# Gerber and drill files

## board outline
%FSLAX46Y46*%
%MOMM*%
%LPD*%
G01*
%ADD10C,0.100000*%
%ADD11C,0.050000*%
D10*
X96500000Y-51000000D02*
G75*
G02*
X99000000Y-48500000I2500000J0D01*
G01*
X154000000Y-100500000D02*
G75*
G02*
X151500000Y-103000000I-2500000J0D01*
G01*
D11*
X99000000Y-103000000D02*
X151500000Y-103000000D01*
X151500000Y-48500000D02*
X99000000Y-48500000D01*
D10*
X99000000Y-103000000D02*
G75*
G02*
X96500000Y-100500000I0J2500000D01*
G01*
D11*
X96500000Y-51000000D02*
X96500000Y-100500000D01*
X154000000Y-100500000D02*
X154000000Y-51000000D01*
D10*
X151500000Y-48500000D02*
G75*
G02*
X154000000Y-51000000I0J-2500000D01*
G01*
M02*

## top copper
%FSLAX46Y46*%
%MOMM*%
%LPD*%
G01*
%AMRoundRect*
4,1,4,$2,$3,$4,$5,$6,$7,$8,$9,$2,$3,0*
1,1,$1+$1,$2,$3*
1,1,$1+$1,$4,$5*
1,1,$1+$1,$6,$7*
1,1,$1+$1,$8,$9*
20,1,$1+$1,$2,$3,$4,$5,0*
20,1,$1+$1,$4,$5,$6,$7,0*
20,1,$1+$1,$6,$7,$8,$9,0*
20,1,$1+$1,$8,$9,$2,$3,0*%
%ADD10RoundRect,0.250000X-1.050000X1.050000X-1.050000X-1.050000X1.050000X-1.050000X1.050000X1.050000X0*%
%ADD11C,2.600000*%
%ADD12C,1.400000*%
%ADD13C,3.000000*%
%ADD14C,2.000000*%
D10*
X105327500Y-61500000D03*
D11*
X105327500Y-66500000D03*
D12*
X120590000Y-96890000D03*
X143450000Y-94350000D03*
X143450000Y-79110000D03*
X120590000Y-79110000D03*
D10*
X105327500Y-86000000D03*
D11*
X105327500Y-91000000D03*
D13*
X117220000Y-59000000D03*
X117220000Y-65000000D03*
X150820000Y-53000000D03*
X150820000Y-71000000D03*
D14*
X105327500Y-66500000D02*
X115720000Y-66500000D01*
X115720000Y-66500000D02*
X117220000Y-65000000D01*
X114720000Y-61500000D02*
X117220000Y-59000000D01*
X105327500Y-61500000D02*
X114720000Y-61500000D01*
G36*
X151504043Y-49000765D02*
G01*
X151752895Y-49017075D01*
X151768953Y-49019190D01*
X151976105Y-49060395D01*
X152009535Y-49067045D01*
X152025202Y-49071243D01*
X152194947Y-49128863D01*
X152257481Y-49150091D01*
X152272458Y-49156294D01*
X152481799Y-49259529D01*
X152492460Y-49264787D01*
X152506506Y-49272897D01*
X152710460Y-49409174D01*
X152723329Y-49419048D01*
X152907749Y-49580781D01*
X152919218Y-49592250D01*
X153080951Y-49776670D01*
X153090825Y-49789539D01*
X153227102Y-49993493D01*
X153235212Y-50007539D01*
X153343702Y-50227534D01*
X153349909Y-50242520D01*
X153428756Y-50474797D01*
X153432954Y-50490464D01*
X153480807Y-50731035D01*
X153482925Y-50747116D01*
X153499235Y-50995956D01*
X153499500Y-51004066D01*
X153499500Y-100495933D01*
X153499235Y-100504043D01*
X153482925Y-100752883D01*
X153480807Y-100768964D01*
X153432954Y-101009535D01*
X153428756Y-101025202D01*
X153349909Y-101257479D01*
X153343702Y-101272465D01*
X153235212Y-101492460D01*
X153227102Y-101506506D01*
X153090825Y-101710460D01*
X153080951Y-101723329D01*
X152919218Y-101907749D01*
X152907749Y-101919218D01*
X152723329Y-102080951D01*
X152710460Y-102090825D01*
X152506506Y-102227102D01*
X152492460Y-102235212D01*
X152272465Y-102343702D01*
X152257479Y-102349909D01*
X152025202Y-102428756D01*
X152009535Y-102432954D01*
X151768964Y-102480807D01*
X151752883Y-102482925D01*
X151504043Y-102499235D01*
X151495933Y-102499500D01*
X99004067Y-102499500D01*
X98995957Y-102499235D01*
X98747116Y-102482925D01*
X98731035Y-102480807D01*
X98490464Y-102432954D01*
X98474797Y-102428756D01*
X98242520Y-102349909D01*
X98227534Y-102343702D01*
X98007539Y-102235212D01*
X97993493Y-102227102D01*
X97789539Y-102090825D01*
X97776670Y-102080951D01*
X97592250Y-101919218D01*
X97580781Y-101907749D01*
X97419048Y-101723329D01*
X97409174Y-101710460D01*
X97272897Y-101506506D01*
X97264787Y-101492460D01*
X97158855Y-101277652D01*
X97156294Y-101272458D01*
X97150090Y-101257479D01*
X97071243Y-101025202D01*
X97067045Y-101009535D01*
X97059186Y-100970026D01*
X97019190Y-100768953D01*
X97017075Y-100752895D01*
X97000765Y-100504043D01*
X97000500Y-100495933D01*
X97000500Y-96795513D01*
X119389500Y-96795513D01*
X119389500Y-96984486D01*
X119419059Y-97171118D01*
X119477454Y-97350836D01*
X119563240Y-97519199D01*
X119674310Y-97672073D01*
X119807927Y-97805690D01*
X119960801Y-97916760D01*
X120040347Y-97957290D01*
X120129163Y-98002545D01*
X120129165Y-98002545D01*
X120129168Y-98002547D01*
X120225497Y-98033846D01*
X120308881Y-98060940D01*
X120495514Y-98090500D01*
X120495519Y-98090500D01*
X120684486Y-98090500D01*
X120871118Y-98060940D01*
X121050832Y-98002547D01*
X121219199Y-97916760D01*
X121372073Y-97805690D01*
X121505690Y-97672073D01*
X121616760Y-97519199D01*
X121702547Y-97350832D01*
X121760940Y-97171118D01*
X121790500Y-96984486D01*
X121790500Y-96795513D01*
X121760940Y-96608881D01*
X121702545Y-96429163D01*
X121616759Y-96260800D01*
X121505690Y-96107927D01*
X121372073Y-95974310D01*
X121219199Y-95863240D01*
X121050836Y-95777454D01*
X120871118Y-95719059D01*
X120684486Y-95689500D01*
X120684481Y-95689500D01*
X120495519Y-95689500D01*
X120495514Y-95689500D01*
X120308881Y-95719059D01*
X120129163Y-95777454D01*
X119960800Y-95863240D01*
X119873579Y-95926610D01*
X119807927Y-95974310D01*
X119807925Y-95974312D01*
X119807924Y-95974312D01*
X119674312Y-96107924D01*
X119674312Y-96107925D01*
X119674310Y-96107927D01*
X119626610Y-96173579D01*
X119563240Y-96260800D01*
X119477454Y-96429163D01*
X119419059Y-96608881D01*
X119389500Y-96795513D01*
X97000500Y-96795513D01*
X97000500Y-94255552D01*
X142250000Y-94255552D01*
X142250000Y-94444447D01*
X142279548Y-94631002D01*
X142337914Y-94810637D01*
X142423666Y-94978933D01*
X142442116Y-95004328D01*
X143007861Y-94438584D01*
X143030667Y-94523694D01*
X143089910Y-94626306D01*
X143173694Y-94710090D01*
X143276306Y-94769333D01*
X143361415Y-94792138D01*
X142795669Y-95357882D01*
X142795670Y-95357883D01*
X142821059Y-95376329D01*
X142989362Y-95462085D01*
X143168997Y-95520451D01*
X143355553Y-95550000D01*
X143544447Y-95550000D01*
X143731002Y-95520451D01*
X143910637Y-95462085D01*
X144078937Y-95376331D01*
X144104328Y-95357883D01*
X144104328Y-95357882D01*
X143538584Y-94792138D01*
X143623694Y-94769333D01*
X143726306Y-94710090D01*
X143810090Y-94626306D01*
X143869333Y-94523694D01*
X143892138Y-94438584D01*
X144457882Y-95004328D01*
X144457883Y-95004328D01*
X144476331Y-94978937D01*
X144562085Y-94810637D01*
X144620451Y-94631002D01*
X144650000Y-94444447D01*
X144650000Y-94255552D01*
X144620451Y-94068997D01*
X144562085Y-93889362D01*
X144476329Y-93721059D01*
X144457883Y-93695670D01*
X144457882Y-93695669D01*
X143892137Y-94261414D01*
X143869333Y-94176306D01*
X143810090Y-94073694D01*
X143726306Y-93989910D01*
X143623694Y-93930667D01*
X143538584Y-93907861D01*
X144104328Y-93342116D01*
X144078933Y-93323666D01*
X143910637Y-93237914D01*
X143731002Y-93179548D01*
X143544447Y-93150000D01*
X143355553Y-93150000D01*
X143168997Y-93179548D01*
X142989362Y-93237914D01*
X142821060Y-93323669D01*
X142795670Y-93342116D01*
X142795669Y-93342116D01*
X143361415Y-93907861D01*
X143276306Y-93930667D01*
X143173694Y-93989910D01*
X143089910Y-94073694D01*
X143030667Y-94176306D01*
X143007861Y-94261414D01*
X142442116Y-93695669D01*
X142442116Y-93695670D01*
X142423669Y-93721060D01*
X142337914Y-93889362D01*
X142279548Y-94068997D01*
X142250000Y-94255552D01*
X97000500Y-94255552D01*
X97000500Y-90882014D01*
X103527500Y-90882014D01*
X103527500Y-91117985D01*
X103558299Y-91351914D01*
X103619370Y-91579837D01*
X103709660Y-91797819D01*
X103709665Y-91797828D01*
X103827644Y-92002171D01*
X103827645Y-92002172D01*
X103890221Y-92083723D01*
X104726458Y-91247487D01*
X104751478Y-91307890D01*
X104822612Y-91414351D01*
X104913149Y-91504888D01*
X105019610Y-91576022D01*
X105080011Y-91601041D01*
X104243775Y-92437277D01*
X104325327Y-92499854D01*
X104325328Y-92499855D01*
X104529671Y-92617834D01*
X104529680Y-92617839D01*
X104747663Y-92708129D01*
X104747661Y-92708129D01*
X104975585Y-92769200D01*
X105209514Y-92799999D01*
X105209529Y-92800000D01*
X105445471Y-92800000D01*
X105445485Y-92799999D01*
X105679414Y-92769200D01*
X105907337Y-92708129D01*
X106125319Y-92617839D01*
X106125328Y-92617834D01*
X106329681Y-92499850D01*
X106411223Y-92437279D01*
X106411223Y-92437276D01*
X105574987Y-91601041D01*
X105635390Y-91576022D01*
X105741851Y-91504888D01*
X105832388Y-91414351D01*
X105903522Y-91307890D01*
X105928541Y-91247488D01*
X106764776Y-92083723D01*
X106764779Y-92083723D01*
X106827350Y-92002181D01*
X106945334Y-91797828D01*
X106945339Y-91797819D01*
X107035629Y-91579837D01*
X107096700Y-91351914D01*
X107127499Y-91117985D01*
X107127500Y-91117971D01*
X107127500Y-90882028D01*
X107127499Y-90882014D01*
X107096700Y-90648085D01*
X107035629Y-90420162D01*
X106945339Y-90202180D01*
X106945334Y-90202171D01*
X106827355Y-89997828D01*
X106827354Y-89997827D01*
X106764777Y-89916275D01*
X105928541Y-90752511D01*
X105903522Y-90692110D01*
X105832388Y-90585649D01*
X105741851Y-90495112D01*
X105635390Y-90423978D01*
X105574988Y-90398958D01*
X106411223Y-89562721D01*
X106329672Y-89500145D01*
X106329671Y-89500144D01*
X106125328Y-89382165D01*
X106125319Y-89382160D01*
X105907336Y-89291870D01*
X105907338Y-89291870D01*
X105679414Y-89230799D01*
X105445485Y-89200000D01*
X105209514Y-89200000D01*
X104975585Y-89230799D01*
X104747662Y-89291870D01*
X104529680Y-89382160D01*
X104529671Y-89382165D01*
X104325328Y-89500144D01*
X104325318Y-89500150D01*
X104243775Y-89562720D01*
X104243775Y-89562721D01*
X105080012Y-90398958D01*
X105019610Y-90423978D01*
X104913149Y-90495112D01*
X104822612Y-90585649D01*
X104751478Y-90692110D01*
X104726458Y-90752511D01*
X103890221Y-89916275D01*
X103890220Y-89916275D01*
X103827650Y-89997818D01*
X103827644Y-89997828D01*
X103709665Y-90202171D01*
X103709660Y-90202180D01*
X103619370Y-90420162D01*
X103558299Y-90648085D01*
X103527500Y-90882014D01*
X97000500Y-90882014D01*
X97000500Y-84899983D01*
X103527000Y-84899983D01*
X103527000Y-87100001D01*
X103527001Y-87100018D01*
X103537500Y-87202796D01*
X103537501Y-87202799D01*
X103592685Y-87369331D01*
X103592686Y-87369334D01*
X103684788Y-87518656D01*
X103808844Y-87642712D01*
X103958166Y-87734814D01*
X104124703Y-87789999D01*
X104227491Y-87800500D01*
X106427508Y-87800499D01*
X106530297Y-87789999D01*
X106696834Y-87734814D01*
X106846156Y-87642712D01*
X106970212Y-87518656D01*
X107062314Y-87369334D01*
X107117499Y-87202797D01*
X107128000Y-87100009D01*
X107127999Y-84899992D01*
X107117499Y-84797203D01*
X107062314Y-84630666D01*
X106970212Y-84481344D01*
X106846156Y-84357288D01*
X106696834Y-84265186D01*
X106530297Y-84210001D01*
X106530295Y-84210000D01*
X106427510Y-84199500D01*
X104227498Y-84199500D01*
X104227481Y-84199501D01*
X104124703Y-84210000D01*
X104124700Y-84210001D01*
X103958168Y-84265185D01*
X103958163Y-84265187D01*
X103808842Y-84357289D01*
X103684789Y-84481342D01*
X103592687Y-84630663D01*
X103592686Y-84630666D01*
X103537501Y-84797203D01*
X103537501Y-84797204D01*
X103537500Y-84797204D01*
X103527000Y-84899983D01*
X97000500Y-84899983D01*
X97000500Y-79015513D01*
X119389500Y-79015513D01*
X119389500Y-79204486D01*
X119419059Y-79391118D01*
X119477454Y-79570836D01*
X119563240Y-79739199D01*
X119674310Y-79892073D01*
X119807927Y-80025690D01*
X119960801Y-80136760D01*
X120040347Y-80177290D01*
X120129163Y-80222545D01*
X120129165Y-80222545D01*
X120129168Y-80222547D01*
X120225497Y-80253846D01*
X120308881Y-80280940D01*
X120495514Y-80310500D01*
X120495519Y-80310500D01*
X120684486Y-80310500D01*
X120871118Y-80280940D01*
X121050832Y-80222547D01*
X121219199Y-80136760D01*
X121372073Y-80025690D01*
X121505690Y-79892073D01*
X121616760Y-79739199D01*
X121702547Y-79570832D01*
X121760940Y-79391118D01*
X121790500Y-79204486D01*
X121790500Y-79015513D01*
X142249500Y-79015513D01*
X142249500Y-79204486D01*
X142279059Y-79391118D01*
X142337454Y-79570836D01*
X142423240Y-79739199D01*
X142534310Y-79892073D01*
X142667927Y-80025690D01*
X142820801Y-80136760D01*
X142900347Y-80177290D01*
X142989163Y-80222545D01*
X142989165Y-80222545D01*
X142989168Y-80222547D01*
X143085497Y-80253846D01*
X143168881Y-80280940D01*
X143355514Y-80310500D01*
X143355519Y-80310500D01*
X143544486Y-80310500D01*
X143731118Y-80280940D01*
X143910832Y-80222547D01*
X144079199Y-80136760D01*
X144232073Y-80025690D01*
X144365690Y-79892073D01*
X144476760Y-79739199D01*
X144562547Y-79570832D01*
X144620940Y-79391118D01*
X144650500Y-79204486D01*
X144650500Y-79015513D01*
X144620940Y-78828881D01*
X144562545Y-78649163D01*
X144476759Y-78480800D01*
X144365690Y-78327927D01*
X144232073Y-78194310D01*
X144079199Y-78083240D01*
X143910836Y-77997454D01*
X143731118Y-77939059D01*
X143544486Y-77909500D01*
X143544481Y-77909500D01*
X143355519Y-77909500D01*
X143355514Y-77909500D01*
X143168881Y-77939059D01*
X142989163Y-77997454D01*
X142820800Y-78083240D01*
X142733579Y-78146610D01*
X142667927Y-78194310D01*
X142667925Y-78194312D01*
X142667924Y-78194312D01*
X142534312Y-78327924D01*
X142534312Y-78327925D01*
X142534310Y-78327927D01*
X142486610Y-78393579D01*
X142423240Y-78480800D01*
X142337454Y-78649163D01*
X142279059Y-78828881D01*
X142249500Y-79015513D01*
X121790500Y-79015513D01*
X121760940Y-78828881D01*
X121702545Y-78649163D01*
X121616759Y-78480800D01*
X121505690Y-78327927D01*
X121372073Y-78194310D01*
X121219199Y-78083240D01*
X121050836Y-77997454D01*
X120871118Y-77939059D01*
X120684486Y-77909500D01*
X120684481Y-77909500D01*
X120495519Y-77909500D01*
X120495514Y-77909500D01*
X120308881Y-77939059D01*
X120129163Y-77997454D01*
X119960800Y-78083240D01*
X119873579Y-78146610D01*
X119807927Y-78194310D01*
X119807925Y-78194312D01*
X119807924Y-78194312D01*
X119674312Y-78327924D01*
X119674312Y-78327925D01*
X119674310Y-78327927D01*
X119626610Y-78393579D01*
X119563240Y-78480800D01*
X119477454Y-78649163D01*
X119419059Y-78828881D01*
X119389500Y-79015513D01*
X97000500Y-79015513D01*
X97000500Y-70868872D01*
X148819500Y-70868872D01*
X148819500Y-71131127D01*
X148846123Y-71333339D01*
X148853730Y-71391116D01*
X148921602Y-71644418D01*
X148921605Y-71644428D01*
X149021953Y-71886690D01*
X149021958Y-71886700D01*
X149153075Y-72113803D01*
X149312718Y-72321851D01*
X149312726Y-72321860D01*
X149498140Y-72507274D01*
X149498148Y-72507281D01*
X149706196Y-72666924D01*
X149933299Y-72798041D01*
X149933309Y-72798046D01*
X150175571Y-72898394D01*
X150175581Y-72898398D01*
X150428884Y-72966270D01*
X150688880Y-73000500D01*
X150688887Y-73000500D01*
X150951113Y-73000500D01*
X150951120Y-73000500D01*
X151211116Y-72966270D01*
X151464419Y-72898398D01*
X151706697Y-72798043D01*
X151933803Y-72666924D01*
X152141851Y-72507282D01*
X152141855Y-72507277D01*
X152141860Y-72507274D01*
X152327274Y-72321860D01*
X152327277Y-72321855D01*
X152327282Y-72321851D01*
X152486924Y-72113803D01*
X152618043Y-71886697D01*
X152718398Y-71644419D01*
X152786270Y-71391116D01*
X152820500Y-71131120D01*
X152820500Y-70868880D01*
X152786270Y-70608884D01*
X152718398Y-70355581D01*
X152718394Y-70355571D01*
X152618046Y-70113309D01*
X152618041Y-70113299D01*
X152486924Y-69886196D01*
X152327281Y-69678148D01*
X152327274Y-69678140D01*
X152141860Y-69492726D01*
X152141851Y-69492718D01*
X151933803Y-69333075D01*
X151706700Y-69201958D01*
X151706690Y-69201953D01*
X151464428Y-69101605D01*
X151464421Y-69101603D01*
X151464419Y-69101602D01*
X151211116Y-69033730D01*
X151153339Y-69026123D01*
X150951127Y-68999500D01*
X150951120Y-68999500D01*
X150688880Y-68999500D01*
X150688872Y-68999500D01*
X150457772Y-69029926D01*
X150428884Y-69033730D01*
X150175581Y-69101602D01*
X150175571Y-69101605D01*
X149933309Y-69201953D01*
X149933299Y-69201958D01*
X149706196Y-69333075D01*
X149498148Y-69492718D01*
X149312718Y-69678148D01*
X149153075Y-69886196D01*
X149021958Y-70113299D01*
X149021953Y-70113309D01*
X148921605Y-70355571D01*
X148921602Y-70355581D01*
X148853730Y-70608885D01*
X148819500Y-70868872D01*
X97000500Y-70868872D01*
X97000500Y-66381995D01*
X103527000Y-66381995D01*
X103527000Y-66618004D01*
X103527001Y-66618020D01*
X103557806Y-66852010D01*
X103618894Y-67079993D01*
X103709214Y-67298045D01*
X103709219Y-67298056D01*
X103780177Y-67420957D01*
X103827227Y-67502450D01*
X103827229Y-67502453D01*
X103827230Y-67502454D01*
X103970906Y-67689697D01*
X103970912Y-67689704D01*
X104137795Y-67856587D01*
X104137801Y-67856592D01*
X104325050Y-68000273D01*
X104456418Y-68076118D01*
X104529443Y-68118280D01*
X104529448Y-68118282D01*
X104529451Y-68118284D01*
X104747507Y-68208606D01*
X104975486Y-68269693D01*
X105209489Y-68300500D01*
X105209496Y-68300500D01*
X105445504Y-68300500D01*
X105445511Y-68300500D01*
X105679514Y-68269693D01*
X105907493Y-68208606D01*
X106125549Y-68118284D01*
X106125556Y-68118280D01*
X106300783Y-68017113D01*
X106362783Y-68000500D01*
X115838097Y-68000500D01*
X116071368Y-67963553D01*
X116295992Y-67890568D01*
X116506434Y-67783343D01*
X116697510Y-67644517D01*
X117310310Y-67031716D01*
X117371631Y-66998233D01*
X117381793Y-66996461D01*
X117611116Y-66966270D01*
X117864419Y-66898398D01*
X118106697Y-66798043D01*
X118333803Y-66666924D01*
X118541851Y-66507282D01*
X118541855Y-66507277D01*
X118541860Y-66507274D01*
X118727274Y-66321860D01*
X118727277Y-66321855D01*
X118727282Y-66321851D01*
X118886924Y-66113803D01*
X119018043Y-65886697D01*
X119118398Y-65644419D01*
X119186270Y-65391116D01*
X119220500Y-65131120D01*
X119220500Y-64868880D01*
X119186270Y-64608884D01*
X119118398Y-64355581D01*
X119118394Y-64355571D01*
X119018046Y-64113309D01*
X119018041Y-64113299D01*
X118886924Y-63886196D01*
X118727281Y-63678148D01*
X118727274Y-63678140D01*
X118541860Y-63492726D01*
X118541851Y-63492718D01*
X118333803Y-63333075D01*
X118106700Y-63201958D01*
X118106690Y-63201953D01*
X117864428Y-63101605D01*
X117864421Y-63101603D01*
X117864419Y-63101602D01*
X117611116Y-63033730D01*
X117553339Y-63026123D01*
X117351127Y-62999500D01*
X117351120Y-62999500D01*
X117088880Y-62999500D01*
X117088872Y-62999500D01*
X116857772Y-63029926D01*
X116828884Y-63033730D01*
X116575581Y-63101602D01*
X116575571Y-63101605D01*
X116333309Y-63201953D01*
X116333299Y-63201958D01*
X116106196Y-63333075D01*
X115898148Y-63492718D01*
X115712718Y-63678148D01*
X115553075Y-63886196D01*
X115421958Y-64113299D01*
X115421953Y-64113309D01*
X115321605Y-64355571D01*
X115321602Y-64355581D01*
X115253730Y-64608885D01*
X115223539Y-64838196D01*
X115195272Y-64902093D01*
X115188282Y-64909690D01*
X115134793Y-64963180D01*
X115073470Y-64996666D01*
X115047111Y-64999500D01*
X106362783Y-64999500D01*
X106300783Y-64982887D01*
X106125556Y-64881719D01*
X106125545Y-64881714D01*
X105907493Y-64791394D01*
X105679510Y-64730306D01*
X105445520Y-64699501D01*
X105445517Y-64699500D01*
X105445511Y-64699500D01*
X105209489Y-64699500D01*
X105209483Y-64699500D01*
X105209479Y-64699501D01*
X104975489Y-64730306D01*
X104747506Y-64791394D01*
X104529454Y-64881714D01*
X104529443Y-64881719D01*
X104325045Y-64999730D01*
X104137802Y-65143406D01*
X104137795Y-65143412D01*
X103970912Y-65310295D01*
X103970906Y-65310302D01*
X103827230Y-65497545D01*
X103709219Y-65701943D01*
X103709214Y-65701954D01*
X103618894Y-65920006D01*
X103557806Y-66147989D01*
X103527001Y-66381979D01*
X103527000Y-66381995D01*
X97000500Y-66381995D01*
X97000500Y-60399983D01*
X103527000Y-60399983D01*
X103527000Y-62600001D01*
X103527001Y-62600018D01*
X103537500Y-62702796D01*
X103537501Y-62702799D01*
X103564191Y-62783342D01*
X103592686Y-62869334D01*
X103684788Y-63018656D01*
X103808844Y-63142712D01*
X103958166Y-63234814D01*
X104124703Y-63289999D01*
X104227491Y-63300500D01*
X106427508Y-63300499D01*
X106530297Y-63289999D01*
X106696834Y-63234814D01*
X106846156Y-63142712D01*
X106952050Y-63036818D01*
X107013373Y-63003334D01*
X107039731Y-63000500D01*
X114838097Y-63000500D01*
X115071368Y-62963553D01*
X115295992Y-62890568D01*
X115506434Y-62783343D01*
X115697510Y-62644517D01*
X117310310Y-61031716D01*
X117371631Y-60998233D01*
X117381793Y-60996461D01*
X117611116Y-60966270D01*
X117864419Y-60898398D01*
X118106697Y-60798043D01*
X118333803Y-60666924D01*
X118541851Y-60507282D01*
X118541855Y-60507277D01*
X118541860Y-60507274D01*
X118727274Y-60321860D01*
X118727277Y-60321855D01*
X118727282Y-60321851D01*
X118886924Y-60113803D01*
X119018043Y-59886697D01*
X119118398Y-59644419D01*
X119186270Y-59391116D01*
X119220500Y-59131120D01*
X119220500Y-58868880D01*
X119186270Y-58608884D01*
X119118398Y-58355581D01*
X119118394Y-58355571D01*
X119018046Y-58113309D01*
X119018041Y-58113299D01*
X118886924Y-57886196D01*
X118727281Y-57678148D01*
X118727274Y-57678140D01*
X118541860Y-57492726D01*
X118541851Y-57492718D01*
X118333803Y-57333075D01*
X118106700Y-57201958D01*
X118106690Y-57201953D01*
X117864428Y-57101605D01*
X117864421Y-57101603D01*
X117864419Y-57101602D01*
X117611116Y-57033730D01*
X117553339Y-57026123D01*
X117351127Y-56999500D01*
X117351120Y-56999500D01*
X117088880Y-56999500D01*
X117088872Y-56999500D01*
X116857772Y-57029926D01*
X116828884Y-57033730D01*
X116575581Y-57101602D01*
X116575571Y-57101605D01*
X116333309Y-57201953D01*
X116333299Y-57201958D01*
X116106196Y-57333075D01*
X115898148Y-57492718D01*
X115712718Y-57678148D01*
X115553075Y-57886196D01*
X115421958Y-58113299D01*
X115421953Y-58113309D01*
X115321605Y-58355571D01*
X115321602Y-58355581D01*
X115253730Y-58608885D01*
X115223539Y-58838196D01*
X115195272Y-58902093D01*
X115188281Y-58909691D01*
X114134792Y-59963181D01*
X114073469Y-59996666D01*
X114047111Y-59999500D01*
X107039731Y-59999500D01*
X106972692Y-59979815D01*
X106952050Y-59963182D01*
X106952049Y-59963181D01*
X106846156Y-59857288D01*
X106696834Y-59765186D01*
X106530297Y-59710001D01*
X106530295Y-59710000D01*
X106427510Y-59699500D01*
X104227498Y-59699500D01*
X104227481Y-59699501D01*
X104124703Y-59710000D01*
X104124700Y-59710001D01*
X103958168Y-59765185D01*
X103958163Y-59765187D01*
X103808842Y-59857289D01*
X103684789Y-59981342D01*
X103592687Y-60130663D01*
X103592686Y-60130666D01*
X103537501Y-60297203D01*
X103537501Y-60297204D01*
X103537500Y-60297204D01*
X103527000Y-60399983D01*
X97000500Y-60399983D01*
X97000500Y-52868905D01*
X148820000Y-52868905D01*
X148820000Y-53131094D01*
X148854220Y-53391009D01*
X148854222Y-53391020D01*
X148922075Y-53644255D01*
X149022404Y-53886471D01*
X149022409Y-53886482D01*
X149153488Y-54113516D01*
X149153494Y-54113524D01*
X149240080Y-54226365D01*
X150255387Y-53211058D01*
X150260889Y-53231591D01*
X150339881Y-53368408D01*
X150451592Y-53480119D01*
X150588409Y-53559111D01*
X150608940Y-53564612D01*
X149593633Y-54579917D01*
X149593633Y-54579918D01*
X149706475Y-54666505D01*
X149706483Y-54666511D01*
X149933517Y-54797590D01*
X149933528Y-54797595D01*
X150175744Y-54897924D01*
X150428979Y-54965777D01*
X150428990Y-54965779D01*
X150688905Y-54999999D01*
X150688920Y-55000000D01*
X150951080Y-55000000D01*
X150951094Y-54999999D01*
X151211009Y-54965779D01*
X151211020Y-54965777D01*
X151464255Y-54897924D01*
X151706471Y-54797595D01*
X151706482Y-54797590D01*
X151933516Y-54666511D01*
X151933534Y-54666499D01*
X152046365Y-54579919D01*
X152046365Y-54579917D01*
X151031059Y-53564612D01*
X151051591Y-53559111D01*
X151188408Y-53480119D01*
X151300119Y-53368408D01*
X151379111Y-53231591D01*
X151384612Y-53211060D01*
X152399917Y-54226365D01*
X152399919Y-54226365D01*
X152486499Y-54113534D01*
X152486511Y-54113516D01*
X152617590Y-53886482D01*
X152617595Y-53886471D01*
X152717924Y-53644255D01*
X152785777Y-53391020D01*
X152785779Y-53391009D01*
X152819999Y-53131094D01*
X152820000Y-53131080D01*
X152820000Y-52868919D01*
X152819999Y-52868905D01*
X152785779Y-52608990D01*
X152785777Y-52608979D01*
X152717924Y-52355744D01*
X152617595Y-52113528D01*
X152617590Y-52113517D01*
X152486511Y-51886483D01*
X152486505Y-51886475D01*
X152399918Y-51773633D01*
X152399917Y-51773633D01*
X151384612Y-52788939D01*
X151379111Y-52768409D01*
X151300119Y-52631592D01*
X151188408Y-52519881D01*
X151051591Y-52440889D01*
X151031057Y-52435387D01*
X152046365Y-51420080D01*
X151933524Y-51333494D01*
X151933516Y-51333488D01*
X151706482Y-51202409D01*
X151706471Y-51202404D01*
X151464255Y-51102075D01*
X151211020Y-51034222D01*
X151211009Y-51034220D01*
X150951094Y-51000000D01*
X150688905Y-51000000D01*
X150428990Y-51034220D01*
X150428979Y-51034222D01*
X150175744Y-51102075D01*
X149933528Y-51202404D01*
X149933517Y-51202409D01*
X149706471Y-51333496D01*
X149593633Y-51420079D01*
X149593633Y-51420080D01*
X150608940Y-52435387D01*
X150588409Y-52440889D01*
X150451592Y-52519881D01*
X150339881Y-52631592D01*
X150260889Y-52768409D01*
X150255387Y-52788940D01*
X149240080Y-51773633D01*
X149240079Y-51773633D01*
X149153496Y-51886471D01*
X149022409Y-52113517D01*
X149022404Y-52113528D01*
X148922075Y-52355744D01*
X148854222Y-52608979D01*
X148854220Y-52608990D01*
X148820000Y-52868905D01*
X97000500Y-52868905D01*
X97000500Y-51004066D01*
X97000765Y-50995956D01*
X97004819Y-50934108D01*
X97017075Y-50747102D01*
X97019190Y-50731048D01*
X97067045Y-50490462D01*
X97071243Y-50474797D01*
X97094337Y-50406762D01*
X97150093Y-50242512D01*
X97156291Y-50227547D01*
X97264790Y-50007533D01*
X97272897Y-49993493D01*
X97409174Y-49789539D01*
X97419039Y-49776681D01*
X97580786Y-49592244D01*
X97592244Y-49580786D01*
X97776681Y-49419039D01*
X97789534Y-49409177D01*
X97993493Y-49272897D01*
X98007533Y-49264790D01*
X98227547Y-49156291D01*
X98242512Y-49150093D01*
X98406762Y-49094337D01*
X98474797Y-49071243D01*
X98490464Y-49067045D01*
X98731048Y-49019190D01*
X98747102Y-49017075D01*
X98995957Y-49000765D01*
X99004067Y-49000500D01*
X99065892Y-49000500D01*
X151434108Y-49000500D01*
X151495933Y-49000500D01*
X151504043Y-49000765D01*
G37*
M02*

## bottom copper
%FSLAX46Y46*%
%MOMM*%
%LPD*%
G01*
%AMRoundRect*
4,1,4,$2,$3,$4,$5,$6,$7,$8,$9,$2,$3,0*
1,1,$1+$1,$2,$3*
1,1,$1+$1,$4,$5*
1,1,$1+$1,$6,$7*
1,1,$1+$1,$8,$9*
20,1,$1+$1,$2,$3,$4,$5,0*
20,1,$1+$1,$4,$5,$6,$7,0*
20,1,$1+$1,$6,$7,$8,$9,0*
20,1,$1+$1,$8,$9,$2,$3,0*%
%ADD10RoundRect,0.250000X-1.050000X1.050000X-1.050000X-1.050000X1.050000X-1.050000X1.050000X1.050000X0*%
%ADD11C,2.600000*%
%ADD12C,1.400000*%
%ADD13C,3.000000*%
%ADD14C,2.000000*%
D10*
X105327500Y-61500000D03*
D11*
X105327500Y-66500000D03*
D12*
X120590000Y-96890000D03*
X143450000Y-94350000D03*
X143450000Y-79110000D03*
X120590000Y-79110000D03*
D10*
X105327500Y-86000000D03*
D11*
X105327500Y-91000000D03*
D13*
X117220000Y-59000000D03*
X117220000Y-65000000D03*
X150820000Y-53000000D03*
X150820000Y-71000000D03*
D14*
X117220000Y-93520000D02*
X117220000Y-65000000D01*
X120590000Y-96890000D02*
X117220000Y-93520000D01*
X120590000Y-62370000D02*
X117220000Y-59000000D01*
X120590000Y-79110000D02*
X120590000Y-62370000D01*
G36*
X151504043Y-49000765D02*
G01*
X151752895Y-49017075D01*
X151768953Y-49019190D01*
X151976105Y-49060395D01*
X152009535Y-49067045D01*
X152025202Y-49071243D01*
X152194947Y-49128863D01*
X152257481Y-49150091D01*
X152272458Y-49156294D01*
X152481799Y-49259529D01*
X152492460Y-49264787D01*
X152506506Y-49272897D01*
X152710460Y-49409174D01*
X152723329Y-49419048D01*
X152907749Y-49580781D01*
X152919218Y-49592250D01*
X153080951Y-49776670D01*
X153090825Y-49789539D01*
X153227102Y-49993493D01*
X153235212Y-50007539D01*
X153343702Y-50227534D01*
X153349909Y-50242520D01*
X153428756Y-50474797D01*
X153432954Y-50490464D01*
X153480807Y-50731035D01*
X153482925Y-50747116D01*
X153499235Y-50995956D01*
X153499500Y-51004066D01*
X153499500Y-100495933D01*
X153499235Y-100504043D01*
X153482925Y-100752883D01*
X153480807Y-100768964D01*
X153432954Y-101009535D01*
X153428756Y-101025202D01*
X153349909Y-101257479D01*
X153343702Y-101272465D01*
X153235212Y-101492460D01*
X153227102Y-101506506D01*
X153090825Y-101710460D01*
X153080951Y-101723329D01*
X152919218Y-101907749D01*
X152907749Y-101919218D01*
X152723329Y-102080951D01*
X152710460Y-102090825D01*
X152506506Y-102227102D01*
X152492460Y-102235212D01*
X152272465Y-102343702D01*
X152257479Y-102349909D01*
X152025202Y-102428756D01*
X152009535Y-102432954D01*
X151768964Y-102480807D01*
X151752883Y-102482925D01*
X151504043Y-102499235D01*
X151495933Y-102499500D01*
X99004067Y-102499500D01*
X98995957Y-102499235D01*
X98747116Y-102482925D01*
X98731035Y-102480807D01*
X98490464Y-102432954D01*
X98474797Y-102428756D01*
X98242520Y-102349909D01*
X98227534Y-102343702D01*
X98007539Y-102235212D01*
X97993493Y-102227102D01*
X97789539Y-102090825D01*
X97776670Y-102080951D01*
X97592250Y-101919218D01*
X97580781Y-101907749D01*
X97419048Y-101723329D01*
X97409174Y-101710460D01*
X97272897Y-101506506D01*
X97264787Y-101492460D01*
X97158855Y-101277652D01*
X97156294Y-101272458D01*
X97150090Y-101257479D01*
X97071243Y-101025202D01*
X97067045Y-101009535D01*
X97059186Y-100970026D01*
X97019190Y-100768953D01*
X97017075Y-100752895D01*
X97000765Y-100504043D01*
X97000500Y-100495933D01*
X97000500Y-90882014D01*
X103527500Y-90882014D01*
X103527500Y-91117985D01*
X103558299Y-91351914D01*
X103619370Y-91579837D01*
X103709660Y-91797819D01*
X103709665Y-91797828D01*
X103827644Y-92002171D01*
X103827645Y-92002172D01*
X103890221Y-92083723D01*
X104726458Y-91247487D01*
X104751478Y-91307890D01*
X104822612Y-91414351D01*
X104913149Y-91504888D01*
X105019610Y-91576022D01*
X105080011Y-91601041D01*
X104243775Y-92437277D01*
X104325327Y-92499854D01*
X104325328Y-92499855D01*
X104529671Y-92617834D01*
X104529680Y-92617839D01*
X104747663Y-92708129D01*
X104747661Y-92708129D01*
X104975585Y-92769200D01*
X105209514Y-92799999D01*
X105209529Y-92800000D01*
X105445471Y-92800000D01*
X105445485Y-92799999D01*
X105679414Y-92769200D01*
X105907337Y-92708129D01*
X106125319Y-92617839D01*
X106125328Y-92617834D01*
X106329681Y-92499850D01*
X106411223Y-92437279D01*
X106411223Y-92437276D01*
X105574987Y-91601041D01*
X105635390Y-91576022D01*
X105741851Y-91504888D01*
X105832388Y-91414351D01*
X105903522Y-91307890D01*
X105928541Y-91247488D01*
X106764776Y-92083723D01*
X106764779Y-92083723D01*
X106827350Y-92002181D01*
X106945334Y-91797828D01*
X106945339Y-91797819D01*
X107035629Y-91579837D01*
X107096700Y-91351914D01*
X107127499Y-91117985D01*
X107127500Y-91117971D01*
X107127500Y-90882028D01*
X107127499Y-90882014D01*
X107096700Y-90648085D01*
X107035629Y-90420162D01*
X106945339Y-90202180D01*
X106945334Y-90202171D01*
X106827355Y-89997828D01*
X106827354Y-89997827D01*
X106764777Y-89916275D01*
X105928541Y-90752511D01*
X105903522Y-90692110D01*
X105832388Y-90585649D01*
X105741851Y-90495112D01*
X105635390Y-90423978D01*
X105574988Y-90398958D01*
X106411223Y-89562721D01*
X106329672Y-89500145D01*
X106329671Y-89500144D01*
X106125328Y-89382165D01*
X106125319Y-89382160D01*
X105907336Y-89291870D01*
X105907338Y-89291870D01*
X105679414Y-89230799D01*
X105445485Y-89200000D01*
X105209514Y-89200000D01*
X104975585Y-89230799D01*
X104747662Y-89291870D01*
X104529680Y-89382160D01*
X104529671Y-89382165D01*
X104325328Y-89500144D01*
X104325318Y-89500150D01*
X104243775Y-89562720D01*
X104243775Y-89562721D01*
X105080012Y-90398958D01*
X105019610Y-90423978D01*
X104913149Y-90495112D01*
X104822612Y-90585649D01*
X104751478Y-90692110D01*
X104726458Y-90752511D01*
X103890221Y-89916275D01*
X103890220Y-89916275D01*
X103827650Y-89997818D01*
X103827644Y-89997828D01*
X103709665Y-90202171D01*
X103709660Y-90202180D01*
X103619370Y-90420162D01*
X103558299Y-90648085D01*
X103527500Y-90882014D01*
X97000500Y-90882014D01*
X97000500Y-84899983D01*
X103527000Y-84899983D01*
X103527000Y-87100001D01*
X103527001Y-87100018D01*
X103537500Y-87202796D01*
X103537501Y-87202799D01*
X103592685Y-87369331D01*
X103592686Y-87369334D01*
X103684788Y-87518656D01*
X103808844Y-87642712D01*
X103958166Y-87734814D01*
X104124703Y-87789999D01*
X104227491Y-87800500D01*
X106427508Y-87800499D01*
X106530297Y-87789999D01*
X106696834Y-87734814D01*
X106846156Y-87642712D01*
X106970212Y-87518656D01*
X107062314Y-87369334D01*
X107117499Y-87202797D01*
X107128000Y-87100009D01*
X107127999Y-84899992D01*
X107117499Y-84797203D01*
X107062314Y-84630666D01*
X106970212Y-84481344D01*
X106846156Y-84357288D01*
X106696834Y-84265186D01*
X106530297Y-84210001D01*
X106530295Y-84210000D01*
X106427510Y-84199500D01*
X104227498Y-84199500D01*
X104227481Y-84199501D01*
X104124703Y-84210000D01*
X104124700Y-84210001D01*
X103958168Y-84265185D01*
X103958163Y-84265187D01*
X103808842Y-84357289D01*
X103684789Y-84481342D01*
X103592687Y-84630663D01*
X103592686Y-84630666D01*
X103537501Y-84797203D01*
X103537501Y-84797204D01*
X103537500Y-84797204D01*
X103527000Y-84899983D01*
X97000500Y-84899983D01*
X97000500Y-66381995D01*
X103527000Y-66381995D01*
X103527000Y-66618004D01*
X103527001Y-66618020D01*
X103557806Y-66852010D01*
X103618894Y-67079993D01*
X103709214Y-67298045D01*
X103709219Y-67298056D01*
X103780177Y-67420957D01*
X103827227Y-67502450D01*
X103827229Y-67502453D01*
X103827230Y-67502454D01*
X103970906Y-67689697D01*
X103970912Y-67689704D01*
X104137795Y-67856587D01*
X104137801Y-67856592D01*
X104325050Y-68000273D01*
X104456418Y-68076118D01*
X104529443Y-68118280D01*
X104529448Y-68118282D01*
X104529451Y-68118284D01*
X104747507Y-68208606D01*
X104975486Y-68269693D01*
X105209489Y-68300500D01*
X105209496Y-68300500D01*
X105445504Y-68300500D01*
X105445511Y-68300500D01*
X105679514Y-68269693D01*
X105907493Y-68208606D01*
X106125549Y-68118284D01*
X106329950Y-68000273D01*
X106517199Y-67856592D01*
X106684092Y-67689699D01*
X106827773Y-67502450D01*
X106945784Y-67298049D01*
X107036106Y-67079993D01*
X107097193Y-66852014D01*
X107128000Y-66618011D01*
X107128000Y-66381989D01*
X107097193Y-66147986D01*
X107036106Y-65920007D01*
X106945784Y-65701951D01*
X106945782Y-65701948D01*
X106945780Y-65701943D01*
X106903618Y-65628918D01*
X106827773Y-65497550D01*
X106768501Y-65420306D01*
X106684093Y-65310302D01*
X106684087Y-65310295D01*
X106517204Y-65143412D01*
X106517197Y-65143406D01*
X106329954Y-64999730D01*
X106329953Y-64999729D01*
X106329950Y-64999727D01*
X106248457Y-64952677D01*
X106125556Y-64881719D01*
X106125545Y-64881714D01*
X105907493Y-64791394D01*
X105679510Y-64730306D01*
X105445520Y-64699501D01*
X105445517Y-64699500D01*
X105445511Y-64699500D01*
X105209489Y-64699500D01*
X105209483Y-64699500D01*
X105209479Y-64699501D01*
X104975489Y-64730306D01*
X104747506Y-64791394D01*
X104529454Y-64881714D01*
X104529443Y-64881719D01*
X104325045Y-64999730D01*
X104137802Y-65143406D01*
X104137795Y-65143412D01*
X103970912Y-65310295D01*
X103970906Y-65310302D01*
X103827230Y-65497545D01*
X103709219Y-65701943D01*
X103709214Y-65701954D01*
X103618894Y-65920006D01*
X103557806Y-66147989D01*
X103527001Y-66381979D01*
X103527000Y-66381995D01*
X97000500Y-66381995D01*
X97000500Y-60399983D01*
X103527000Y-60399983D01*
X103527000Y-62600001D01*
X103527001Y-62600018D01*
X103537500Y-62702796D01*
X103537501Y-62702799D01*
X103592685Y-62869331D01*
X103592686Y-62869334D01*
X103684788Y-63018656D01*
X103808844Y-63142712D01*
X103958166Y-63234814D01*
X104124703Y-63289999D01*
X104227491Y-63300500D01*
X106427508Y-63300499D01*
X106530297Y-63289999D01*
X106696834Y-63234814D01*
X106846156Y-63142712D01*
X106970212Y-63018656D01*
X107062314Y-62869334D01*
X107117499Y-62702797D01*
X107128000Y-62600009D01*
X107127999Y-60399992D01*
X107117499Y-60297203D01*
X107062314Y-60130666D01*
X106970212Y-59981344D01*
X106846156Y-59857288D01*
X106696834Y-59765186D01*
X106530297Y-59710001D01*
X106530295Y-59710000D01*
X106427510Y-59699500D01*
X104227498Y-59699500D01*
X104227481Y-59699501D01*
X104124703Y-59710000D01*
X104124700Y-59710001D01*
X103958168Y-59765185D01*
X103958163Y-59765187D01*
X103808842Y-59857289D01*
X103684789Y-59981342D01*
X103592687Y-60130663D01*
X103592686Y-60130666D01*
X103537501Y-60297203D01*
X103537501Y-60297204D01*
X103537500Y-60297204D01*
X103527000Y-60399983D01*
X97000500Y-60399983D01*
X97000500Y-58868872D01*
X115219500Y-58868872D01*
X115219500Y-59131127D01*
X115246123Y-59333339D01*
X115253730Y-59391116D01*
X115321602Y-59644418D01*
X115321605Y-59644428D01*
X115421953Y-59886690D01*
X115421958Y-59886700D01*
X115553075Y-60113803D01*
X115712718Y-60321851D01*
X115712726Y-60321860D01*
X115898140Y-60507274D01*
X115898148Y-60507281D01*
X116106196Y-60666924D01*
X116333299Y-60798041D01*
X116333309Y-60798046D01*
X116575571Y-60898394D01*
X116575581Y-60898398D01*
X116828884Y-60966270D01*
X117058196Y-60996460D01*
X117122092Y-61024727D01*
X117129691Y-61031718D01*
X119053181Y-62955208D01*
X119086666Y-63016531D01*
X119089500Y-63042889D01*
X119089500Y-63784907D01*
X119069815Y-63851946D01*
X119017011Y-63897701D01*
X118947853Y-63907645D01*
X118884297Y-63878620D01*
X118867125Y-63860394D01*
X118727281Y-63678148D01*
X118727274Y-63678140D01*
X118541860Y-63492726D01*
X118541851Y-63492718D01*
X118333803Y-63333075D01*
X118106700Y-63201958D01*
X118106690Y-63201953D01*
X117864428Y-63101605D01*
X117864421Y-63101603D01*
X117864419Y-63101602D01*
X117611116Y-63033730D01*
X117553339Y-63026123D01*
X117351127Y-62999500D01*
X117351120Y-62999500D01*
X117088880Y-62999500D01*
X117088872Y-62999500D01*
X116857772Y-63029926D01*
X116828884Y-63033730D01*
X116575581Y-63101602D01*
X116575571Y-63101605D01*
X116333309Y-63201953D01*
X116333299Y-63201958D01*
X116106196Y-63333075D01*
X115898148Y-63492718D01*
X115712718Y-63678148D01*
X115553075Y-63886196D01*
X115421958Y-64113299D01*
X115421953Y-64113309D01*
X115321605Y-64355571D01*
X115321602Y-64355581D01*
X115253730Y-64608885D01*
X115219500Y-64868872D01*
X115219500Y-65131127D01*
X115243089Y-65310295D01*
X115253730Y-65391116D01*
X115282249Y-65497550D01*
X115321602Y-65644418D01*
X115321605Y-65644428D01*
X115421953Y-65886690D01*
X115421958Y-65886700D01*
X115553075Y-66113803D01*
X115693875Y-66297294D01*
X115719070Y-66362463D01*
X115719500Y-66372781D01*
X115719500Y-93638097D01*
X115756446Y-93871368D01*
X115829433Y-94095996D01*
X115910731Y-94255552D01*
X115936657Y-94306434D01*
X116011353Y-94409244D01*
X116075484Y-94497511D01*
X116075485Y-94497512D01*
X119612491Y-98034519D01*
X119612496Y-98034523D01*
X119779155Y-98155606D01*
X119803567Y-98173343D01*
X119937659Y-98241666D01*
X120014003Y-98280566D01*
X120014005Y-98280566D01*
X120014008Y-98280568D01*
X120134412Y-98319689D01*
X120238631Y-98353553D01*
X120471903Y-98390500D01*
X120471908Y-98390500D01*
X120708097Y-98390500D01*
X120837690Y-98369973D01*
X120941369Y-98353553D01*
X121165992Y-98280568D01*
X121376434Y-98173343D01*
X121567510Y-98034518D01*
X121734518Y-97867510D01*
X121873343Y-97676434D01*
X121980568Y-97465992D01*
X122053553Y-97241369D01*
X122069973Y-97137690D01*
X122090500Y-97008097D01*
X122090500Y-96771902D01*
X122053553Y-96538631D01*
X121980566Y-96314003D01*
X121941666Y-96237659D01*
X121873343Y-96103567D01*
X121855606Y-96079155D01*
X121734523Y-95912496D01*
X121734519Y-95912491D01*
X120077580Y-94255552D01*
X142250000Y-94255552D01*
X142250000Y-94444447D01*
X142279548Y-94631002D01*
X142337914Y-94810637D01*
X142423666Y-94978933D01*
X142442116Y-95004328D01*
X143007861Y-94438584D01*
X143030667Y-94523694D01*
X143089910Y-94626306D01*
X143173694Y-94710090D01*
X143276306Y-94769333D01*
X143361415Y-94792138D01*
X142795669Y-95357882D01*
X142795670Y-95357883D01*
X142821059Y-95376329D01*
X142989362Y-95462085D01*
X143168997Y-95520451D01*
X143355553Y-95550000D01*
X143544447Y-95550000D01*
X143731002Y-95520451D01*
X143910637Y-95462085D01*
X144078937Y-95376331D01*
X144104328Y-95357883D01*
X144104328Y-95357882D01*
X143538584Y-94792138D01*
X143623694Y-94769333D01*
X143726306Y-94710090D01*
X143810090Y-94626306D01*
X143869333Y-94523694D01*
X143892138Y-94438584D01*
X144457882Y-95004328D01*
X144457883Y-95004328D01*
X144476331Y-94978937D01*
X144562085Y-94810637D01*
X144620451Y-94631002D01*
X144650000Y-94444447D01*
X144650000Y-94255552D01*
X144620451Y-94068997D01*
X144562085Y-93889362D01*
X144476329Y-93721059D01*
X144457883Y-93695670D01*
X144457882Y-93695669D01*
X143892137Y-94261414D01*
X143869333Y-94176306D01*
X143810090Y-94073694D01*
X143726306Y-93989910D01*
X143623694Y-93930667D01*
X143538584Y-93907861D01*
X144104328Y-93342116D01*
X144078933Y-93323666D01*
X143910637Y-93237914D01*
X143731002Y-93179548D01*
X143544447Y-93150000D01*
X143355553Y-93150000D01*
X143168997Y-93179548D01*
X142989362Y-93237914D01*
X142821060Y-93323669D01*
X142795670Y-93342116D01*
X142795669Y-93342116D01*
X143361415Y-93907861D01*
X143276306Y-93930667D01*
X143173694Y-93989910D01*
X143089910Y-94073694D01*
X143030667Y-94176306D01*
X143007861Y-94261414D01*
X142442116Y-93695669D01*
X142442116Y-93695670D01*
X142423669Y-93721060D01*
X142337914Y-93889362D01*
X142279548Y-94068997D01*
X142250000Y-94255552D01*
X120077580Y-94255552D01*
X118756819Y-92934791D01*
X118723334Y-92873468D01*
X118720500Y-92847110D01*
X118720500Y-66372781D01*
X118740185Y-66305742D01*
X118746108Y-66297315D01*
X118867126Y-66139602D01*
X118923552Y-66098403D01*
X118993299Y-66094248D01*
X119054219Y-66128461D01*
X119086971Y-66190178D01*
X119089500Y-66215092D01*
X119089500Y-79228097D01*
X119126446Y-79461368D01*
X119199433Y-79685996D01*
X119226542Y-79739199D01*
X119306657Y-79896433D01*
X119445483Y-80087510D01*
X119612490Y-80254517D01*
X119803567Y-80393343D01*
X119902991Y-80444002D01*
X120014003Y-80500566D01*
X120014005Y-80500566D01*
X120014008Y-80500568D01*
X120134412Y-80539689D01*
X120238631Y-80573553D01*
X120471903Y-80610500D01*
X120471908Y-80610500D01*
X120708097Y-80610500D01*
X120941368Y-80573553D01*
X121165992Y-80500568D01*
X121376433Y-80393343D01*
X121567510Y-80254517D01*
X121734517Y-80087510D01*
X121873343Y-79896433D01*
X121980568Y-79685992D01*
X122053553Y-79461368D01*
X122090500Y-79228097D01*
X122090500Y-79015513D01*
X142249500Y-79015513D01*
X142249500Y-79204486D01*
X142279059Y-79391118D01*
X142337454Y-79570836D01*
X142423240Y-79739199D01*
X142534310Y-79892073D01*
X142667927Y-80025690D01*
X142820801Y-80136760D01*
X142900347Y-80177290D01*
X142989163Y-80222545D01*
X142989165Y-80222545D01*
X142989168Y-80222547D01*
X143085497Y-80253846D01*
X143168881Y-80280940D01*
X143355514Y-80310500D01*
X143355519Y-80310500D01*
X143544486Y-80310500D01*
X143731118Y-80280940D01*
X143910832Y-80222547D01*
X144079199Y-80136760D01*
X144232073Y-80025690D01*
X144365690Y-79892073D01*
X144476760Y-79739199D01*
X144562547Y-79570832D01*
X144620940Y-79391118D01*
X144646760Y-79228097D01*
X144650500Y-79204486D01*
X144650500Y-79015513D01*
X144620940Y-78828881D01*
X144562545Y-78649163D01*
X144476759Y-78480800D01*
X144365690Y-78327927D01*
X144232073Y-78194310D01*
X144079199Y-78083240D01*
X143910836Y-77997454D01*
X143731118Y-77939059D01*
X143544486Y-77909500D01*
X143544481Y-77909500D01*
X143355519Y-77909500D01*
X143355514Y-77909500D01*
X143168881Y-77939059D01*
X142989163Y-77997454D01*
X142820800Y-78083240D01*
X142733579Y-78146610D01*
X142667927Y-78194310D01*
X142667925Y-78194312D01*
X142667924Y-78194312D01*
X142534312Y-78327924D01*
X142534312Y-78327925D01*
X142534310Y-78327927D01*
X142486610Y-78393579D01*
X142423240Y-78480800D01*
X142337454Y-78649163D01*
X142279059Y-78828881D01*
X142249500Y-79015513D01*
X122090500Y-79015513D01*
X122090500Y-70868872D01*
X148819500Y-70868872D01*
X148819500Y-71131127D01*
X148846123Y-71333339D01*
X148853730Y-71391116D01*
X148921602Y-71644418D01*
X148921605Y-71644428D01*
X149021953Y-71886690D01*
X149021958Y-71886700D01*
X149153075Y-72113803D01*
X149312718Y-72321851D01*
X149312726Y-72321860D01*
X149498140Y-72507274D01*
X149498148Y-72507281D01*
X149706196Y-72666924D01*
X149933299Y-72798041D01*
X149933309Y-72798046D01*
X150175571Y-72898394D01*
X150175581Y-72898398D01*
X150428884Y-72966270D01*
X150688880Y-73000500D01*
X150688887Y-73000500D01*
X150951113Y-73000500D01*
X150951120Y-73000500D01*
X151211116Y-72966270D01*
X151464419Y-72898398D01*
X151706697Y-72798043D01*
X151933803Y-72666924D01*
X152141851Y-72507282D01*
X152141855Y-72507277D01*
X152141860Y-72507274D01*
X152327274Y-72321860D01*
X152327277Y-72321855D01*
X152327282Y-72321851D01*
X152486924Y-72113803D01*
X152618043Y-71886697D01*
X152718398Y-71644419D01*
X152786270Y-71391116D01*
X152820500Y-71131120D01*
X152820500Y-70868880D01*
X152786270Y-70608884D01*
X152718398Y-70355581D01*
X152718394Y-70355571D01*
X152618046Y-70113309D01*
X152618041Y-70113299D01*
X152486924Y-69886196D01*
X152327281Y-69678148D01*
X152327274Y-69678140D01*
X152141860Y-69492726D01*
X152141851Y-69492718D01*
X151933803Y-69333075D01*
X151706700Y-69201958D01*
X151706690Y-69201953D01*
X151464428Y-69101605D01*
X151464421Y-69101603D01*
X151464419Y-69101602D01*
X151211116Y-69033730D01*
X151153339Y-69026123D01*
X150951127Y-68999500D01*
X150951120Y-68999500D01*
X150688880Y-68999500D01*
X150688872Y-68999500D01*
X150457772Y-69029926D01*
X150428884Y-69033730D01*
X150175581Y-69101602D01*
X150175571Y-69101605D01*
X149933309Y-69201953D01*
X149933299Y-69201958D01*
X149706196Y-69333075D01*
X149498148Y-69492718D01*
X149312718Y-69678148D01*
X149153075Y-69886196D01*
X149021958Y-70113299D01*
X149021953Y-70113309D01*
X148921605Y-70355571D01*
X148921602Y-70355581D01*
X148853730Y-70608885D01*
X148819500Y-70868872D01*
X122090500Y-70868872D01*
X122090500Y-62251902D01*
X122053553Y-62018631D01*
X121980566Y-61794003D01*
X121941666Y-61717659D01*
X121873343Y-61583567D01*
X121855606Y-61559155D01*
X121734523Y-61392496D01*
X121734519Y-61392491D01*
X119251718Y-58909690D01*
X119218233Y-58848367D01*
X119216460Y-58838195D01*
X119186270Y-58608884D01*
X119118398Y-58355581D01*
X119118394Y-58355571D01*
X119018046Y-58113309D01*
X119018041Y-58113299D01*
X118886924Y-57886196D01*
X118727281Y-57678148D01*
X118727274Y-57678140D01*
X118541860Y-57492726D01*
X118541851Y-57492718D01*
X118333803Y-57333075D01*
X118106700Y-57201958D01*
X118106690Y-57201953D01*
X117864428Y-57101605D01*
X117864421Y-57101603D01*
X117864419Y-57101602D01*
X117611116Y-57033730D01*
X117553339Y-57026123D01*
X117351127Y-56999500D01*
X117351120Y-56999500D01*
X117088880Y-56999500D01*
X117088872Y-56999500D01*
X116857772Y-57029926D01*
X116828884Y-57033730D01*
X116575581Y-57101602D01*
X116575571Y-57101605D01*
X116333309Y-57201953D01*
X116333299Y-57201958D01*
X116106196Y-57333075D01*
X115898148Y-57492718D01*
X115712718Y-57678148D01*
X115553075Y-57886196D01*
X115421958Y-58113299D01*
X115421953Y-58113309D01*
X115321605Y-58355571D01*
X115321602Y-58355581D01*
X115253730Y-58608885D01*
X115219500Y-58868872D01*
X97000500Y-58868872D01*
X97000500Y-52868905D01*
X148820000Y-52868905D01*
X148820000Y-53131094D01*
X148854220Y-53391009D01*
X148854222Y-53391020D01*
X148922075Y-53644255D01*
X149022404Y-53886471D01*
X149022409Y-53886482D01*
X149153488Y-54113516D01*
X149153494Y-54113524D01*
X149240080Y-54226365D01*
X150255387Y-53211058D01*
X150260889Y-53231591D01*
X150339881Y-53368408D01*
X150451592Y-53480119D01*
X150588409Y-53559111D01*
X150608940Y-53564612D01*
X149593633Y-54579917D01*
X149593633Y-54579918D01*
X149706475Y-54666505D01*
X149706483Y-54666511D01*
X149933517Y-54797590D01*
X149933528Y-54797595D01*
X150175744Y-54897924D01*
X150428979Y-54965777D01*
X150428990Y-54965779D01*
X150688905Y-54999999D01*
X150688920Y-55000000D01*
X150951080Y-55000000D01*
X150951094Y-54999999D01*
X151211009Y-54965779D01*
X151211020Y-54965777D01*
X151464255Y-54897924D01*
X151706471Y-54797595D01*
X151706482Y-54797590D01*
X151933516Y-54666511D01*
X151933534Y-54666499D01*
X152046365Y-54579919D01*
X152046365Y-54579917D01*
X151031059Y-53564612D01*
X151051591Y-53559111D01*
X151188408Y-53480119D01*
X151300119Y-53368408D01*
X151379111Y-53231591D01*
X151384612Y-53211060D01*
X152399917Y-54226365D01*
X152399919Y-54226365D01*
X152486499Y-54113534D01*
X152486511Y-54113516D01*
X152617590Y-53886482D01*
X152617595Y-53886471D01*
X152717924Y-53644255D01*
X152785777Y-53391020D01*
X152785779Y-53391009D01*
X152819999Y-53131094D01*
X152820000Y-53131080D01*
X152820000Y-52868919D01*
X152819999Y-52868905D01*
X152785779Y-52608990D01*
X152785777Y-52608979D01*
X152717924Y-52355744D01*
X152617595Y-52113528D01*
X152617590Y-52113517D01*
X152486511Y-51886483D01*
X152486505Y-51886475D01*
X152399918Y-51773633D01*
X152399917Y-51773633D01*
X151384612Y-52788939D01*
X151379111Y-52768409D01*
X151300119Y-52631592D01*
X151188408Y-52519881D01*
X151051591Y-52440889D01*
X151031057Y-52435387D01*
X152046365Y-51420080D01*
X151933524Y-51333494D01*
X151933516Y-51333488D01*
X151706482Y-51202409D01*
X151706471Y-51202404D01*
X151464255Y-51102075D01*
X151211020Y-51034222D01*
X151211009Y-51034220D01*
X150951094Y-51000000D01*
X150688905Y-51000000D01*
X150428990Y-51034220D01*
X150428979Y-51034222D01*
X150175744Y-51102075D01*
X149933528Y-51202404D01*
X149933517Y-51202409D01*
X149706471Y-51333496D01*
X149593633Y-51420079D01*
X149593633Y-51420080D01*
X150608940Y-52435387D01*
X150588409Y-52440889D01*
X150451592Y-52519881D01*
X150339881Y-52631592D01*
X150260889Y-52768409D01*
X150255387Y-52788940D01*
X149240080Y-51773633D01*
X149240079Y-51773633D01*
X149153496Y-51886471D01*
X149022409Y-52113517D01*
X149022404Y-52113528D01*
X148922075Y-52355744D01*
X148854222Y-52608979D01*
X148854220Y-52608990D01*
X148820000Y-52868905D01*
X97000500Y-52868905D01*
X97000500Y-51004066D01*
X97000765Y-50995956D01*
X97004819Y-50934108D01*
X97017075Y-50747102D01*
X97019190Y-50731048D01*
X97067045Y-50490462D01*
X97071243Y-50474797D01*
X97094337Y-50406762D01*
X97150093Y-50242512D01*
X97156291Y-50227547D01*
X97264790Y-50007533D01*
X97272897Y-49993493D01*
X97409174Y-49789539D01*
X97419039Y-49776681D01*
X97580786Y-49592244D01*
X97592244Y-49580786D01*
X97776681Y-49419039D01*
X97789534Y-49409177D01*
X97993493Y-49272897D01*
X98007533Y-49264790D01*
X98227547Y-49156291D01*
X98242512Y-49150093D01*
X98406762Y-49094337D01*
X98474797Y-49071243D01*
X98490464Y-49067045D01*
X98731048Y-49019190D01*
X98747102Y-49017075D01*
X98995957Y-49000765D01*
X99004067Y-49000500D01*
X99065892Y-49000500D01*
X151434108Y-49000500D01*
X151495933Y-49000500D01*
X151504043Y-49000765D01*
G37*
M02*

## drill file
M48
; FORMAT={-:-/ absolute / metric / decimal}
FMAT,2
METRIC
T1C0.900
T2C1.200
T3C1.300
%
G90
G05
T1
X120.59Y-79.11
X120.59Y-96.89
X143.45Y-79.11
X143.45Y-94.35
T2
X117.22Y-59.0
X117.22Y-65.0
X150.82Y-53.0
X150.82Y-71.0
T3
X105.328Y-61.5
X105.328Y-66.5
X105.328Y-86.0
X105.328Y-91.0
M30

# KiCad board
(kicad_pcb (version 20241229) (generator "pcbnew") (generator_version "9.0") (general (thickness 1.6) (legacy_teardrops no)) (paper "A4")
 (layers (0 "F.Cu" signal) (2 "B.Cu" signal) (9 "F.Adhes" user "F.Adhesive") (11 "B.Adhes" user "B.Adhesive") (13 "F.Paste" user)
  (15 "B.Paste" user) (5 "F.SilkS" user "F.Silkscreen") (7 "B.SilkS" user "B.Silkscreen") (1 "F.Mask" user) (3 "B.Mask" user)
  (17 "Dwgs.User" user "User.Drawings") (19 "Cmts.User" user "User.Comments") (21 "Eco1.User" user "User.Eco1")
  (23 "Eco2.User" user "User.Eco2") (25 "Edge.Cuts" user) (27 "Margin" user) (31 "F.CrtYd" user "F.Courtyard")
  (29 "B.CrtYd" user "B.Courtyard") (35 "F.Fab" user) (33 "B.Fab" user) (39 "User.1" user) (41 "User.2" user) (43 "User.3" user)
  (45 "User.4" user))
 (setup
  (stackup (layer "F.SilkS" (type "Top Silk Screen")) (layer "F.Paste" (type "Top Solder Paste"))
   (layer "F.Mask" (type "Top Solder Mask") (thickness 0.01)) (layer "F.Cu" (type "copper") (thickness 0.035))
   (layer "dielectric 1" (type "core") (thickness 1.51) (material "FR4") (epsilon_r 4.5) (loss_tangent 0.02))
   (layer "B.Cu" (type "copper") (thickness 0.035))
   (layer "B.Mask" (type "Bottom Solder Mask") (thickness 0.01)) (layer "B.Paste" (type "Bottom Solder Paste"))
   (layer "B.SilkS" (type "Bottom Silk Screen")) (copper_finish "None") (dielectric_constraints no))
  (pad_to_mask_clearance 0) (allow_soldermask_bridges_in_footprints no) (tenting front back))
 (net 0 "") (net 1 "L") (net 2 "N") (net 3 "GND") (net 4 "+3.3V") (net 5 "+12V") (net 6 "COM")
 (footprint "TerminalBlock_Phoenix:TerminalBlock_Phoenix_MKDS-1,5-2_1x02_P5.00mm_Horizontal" (layer "F.Cu") (at 105.3275 61.5 -90)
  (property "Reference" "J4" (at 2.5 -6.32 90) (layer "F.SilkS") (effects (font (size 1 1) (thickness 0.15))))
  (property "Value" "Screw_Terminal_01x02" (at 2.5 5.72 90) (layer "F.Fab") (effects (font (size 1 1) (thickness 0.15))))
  (pad "1" thru_hole roundrect (at 0 0 270) (size 2.6 2.6) (drill 1.3) (layers "*.Cu" "*.Mask") (remove_unused_layers no)
   (roundrect_rratio 0.096154) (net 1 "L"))
  (pad "2" thru_hole circle (at 5 0 270) (size 2.6 2.6) (drill 1.3) (layers "*.Cu" "*.Mask") (remove_unused_layers no) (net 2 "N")))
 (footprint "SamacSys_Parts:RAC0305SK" (layer "F.Cu") (at 120.59 96.89)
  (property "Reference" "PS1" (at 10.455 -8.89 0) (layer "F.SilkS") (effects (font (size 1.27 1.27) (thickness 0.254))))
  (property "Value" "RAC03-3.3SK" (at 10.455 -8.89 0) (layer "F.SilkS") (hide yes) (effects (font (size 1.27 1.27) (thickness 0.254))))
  (pad "1" thru_hole circle (at 0 0) (size 1.4 1.4) (drill 0.9) (layers "*.Cu" "*.Mask") (remove_unused_layers no) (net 2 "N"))
  (pad "2" thru_hole circle (at 22.86 -2.54) (size 1.4 1.4) (drill 0.9) (layers "*.Cu" "*.Mask") (remove_unused_layers no) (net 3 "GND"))
  (pad "3" thru_hole circle (at 22.86 -17.78) (size 1.4 1.4) (drill 0.9) (layers "*.Cu" "*.Mask") (remove_unused_layers no) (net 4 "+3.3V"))
  (pad "4" thru_hole circle (at 0 -17.78) (size 1.4 1.4) (drill 0.9) (layers "*.Cu" "*.Mask") (remove_unused_layers no) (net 1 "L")))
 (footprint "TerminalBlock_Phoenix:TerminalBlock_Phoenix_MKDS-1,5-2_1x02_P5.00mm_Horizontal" (layer "F.Cu") (at 105.3275 86 -90)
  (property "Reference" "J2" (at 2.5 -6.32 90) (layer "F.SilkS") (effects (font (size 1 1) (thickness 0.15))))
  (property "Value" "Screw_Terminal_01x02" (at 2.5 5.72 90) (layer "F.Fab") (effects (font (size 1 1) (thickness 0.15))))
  (pad "1" thru_hole roundrect (at 0 0 270) (size 2.6 2.6) (drill 1.3) (layers "*.Cu" "*.Mask") (remove_unused_layers no)
   (roundrect_rratio 0.096154) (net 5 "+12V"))
  (pad "2" thru_hole circle (at 5 0 270) (size 2.6 2.6) (drill 1.3) (layers "*.Cu" "*.Mask") (remove_unused_layers no) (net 3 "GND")))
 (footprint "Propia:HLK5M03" (layer "F.Cu") (at 134 62)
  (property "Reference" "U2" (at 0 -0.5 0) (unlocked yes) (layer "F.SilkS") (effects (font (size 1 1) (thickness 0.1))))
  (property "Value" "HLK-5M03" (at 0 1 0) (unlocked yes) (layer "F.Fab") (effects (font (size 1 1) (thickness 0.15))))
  (pad "1" thru_hole circle (at -16.78 -3) (size 3 3) (drill 1.2) (layers "*.Cu" "*.Mask") (remove_unused_layers no) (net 1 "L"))
  (pad "2" thru_hole circle (at -16.78 3) (size 3 3) (drill 1.2) (layers "*.Cu" "*.Mask") (remove_unused_layers no) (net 2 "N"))
  (pad "3" thru_hole circle (at 16.82 -9) (size 3 3) (drill 1.2) (layers "*.Cu" "*.Mask") (remove_unused_layers no) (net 3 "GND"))
  (pad "4" thru_hole circle (at 16.82 9) (size 3 3) (drill 1.2) (layers "*.Cu" "*.Mask") (remove_unused_layers no) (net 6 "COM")))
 (gr_arc (start 96.5 51) (mid 97.232233 49.232233) (end 99 48.5) (stroke (width 0.1) (type solid)) (layer "Edge.Cuts"))
 (gr_arc (start 154 100.5) (mid 153.267767 102.267767) (end 151.5 103) (stroke (width 0.1) (type solid)) (layer "Edge.Cuts"))
 (gr_line (start 99 103) (end 151.5 103) (stroke (width 0.05) (type default)) (layer "Edge.Cuts"))
 (gr_line (start 151.5 48.5) (end 99 48.5) (stroke (width 0.05) (type default)) (layer "Edge.Cuts"))
 (gr_arc (start 99 103) (mid 97.232233 102.267767) (end 96.5 100.5) (stroke (width 0.1) (type solid)) (layer "Edge.Cuts"))
 (gr_line (start 96.5 51) (end 96.5 100.5) (stroke (width 0.05) (type default)) (layer "Edge.Cuts"))
 (gr_line (start 154 100.5) (end 154 51) (stroke (width 0.05) (type default)) (layer "Edge.Cuts"))
 (gr_arc (start 151.5 48.5) (mid 153.267767 49.232233) (end 154 51) (stroke (width 0.1) (type solid)) (layer "Edge.Cuts"))
 (segment (start 105.3275 66.5) (end 115.72 66.5) (width 2) (layer "F.Cu") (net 2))
 (segment (start 115.72 66.5) (end 117.22 65) (width 2) (layer "F.Cu") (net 2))
 (segment (start 117.22 93.52) (end 117.22 65) (width 2) (layer "B.Cu") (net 2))
 (segment (start 120.59 96.89) (end 117.22 93.52) (width 2) (layer "B.Cu") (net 2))
 (segment (start 114.72 61.5) (end 117.22 59) (width 2) (layer "F.Cu") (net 1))
 (segment (start 105.3275 61.5) (end 114.72 61.5) (width 2) (layer "F.Cu") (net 1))
 (segment (start 120.59 62.37) (end 117.22 59) (width 2) (layer "B.Cu") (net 1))
 (segment (start 120.59 79.11) (end 120.59 62.37) (width 2) (layer "B.Cu") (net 1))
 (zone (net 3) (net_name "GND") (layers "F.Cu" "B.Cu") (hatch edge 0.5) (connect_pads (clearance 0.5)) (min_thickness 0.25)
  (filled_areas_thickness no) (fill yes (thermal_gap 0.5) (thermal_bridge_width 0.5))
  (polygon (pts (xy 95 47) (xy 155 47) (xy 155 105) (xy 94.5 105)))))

